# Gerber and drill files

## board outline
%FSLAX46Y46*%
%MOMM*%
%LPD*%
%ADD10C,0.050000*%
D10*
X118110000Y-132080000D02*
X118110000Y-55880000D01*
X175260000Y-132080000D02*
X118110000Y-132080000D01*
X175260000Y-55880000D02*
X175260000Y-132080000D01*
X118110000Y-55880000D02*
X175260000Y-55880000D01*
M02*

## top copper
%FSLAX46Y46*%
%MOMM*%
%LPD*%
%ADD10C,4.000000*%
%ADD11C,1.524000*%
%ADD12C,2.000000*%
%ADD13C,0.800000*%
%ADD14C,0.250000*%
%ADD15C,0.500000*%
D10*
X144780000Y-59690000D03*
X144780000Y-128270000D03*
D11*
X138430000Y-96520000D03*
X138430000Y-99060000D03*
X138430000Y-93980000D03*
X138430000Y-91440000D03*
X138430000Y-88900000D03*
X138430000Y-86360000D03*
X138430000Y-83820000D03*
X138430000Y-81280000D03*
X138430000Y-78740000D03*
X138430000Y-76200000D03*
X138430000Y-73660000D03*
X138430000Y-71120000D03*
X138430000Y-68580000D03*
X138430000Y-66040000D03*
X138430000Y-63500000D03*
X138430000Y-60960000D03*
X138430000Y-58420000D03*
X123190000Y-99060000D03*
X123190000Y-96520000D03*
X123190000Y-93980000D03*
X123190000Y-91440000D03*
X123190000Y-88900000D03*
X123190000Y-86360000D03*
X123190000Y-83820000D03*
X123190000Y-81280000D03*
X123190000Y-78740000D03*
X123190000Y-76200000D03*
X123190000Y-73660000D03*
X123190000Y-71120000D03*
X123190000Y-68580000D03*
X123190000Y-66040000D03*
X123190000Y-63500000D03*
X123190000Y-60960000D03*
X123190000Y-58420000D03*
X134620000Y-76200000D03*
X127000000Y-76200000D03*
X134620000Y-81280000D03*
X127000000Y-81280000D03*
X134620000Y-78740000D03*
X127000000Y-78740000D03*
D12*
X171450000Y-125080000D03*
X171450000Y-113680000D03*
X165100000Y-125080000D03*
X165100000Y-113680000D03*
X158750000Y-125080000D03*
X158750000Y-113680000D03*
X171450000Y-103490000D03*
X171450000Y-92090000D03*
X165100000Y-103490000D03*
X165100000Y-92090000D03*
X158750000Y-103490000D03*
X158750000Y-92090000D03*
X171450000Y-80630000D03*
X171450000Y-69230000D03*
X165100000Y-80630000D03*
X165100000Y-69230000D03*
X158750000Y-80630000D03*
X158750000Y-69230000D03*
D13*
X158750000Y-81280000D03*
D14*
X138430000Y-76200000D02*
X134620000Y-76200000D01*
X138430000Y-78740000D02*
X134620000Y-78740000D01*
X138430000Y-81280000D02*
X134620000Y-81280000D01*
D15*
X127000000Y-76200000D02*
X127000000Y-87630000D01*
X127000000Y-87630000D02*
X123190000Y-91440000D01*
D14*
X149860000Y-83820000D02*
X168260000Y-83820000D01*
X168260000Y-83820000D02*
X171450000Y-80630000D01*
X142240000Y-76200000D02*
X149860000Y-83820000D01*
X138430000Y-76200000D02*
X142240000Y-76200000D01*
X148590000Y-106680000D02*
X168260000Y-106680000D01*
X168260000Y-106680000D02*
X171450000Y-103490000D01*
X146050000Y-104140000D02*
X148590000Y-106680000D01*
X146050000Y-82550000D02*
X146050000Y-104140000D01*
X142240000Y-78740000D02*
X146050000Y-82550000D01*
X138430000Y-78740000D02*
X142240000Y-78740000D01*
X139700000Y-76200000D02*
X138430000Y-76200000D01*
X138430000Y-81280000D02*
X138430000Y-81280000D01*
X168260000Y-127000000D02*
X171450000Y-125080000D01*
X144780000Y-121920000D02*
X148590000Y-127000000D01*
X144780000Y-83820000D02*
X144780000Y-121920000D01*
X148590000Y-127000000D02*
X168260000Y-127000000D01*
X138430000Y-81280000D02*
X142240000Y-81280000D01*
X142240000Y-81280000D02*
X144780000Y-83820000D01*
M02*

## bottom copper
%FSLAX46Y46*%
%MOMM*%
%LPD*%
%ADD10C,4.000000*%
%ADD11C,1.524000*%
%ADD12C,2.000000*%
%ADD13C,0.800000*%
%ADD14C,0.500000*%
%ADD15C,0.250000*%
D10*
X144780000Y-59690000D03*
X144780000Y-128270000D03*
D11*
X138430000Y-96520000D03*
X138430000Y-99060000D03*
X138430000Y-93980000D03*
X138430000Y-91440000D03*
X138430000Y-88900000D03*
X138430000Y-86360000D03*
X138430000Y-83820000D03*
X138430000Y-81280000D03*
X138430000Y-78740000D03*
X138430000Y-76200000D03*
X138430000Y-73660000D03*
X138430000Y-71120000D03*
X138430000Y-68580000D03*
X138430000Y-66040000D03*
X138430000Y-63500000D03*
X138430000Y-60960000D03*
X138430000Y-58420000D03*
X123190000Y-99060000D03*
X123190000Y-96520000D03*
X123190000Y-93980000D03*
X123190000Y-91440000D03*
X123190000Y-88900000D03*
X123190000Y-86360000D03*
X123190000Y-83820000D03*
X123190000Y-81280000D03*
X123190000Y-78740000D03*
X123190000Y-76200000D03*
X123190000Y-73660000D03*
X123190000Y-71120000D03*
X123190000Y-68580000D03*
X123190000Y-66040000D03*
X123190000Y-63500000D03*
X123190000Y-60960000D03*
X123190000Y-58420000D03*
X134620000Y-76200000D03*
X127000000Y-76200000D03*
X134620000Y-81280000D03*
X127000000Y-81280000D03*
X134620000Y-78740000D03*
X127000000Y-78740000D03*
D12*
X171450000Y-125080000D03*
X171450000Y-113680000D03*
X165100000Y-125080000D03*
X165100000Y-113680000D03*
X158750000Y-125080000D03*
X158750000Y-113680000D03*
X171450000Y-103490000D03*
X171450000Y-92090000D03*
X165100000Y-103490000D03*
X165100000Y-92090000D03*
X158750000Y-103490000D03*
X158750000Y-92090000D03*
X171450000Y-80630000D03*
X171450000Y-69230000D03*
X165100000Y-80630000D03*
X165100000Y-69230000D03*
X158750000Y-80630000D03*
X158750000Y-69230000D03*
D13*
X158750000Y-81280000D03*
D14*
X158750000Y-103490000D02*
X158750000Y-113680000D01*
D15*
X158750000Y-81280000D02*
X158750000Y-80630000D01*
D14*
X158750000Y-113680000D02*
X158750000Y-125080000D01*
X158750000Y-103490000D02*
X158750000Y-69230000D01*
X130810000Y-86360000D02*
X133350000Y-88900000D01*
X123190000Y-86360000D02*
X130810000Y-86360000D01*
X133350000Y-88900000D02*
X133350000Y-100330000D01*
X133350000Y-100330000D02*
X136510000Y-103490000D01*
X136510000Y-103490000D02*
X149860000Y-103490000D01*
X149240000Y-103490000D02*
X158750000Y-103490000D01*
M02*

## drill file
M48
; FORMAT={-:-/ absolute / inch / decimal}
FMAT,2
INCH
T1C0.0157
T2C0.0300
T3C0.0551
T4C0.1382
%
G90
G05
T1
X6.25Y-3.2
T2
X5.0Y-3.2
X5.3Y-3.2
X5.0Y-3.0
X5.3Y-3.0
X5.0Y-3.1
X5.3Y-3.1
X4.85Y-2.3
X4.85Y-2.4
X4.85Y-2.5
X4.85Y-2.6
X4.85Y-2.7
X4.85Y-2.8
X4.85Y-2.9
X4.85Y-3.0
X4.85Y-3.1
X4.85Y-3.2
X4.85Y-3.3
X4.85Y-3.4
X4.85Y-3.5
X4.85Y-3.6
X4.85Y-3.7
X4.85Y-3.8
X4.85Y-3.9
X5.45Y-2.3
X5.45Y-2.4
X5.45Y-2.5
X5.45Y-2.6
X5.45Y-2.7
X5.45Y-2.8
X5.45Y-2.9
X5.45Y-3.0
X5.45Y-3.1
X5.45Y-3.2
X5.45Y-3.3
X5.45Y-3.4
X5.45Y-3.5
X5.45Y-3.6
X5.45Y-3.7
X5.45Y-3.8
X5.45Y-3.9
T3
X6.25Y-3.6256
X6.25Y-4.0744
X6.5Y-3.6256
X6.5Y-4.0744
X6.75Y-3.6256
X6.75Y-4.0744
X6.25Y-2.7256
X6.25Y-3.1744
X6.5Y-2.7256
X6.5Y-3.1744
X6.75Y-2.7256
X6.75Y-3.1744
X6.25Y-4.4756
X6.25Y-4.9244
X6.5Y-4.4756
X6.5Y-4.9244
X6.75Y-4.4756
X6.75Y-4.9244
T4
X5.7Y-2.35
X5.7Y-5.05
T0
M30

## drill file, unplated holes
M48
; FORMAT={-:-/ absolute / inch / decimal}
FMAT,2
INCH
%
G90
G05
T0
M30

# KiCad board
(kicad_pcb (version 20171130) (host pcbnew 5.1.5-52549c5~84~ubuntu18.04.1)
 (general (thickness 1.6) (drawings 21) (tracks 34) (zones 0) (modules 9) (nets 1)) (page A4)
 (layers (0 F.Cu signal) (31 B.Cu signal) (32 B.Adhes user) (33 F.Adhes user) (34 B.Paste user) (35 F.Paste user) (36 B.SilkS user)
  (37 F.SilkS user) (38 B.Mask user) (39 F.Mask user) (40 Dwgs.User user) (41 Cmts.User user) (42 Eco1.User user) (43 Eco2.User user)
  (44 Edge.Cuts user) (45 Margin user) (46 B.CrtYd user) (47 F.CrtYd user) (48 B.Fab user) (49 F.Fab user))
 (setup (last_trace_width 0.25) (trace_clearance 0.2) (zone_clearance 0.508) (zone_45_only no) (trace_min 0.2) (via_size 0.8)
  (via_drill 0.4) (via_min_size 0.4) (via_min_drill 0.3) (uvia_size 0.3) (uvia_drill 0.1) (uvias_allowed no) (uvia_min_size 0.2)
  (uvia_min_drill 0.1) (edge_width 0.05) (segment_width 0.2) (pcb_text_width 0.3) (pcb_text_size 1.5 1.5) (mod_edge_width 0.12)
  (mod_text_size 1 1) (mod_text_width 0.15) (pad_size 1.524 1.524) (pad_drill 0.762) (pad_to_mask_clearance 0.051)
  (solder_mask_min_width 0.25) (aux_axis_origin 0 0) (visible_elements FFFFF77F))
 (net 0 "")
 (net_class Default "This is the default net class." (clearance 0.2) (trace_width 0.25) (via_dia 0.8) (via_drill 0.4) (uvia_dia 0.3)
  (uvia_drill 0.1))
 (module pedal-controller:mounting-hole (layer F.Cu) (at 144.78 59.69)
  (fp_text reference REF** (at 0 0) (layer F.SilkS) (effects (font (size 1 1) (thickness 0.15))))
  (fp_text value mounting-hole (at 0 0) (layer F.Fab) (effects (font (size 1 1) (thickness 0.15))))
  (pad 1 thru_hole circle (at 0 0) (size 4 4) (drill 3.51) (layers *.Cu *.Mask)))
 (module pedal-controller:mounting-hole (layer F.Cu) (at 144.78 128.27)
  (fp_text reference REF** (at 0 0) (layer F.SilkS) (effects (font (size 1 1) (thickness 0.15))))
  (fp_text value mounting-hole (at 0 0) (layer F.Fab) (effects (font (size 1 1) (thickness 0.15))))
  (pad 1 thru_hole circle (at 0 0) (size 4 4) (drill 3.51) (layers *.Cu *.Mask)))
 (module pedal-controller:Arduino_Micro (layer F.Cu) (at 123.19 58.42 270)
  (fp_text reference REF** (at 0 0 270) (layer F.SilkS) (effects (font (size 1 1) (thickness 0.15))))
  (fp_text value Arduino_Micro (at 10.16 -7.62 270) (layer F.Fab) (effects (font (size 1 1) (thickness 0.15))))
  (pad 34 thru_hole circle (at 38.1 -15.24 270) (size 1.524 1.524) (drill 0.762) (layers *.Cu *.Mask))
  (pad 33 thru_hole circle (at 40.64 -15.24 270) (size 1.524 1.524) (drill 0.762) (layers *.Cu *.Mask))
  (pad 32 thru_hole circle (at 35.56 -15.24 270) (size 1.524 1.524) (drill 0.762) (layers *.Cu *.Mask))
  (pad 31 thru_hole circle (at 33.02 -15.24 270) (size 1.524 1.524) (drill 0.762) (layers *.Cu *.Mask))
  (pad 30 thru_hole circle (at 30.48 -15.24 270) (size 1.524 1.524) (drill 0.762) (layers *.Cu *.Mask))
  (pad 29 thru_hole circle (at 27.94 -15.24 270) (size 1.524 1.524) (drill 0.762) (layers *.Cu *.Mask))
  (pad 28 thru_hole circle (at 25.4 -15.24 270) (size 1.524 1.524) (drill 0.762) (layers *.Cu *.Mask))
  (pad 27 thru_hole circle (at 22.86 -15.24 270) (size 1.524 1.524) (drill 0.762) (layers *.Cu *.Mask))
  (pad 26 thru_hole circle (at 20.32 -15.24 270) (size 1.524 1.524) (drill 0.762) (layers *.Cu *.Mask))
  (pad 25 thru_hole circle (at 17.78 -15.24 270) (size 1.524 1.524) (drill 0.762) (layers *.Cu *.Mask))
  (pad 24 thru_hole circle (at 15.24 -15.24 270) (size 1.524 1.524) (drill 0.762) (layers *.Cu *.Mask))
  (pad 23 thru_hole circle (at 12.7 -15.24 270) (size 1.524 1.524) (drill 0.762) (layers *.Cu *.Mask))
  (pad 22 thru_hole circle (at 10.16 -15.24 270) (size 1.524 1.524) (drill 0.762) (layers *.Cu *.Mask))
  (pad 21 thru_hole circle (at 7.62 -15.24 270) (size 1.524 1.524) (drill 0.762) (layers *.Cu *.Mask))
  (pad 20 thru_hole circle (at 5.08 -15.24 270) (size 1.524 1.524) (drill 0.762) (layers *.Cu *.Mask))
  (pad 19 thru_hole circle (at 2.54 -15.24 270) (size 1.524 1.524) (drill 0.762) (layers *.Cu *.Mask))
  (pad 18 thru_hole circle (at 0 -15.24 270) (size 1.524 1.524) (drill 0.762) (layers *.Cu *.Mask))
  (pad 17 thru_hole circle (at 40.64 0 270) (size 1.524 1.524) (drill 0.762) (layers *.Cu *.Mask))
  (pad 16 thru_hole circle (at 38.1 0 270) (size 1.524 1.524) (drill 0.762) (layers *.Cu *.Mask))
  (pad 15 thru_hole circle (at 35.56 0 270) (size 1.524 1.524) (drill 0.762) (layers *.Cu *.Mask))
  (pad 14 thru_hole circle (at 33.02 0 270) (size 1.524 1.524) (drill 0.762) (layers *.Cu *.Mask))
  (pad 13 thru_hole circle (at 30.48 0 270) (size 1.524 1.524) (drill 0.762) (layers *.Cu *.Mask))
  (pad 12 thru_hole circle (at 27.94 0 270) (size 1.524 1.524) (drill 0.762) (layers *.Cu *.Mask))
  (pad 11 thru_hole circle (at 25.4 0 270) (size 1.524 1.524) (drill 0.762) (layers *.Cu *.Mask))
  (pad 10 thru_hole circle (at 22.86 0 270) (size 1.524 1.524) (drill 0.762) (layers *.Cu *.Mask))
  (pad 9 thru_hole circle (at 20.32 0 270) (size 1.524 1.524) (drill 0.762) (layers *.Cu *.Mask))
  (pad 8 thru_hole circle (at 17.78 0 270) (size 1.524 1.524) (drill 0.762) (layers *.Cu *.Mask))
  (pad 7 thru_hole circle (at 15.24 0 270) (size 1.524 1.524) (drill 0.762) (layers *.Cu *.Mask))
  (pad 6 thru_hole circle (at 12.7 0 270) (size 1.524 1.524) (drill 0.762) (layers *.Cu *.Mask))
  (pad 5 thru_hole circle (at 10.16 0 270) (size 1.524 1.524) (drill 0.762) (layers *.Cu *.Mask))
  (pad 4 thru_hole circle (at 7.62 0 270) (size 1.524 1.524) (drill 0.762) (layers *.Cu *.Mask))
  (pad 3 thru_hole circle (at 5.08 0 270) (size 1.524 1.524) (drill 0.762) (layers *.Cu *.Mask))
  (pad 2 thru_hole circle (at 2.54 0 270) (size 1.524 1.524) (drill 0.762) (layers *.Cu *.Mask))
  (pad 1 thru_hole circle (at 0 0 270) (size 1.524 1.524) (drill 0.762) (layers *.Cu *.Mask)))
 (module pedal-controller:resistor (layer F.Cu) (at 127 76.2)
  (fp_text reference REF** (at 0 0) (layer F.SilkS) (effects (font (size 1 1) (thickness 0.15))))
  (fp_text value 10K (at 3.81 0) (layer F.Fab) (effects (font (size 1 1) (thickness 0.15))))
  (pad 2 thru_hole circle (at 7.62 0) (size 1.524 1.524) (drill 0.762) (layers *.Cu *.Mask))
  (pad 1 thru_hole circle (at 0 0) (size 1.524 1.524) (drill 0.762) (layers *.Cu *.Mask)))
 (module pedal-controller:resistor (layer F.Cu) (at 127 81.28)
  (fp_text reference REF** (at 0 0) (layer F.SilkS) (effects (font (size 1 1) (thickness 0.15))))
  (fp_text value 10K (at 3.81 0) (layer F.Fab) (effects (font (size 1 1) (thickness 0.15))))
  (pad 2 thru_hole circle (at 7.62 0) (size 1.524 1.524) (drill 0.762) (layers *.Cu *.Mask))
  (pad 1 thru_hole circle (at 0 0) (size 1.524 1.524) (drill 0.762) (layers *.Cu *.Mask)))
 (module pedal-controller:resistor (layer F.Cu) (at 127 78.74)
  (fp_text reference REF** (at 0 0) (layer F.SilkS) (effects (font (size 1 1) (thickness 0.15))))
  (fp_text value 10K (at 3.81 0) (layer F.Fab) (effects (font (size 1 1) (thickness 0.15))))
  (pad 2 thru_hole circle (at 7.62 0) (size 1.524 1.524) (drill 0.762) (layers *.Cu *.Mask))
  (pad 1 thru_hole circle (at 0 0) (size 1.524 1.524) (drill 0.762) (layers *.Cu *.Mask)))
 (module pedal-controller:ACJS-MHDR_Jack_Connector (layer F.Cu) (at 165.1 119.38)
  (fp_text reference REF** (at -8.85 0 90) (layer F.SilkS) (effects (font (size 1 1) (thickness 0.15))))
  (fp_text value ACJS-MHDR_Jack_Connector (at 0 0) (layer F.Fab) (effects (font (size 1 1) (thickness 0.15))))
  (pad 3 thru_hole circle (at 6.35 5.7) (size 2 2) (drill 1.4) (layers *.Cu *.Mask))
  (pad 4 thru_hole circle (at 6.35 -5.7) (size 2 2) (drill 1.4) (layers *.Cu *.Mask))
  (pad 2 thru_hole circle (at 0 5.7) (size 2 2) (drill 1.4) (layers *.Cu *.Mask))
  (pad 5 thru_hole circle (at 0 -5.7) (size 2 2) (drill 1.4) (layers *.Cu *.Mask))
  (pad 1 thru_hole circle (at -6.35 5.7) (size 2 2) (drill 1.4) (layers *.Cu *.Mask))
  (pad 6 thru_hole circle (at -6.35 -5.7) (size 2 2) (drill 1.4) (layers *.Cu *.Mask)))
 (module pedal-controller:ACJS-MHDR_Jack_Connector (layer F.Cu) (at 165.1 97.79)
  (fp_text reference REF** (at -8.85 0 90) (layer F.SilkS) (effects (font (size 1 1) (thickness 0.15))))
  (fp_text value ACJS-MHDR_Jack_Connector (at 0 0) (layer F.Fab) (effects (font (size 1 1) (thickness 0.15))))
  (pad 3 thru_hole circle (at 6.35 5.7) (size 2 2) (drill 1.4) (layers *.Cu *.Mask))
  (pad 4 thru_hole circle (at 6.35 -5.7) (size 2 2) (drill 1.4) (layers *.Cu *.Mask))
  (pad 2 thru_hole circle (at 0 5.7) (size 2 2) (drill 1.4) (layers *.Cu *.Mask))
  (pad 5 thru_hole circle (at 0 -5.7) (size 2 2) (drill 1.4) (layers *.Cu *.Mask))
  (pad 1 thru_hole circle (at -6.35 5.7) (size 2 2) (drill 1.4) (layers *.Cu *.Mask))
  (pad 6 thru_hole circle (at -6.35 -5.7) (size 2 2) (drill 1.4) (layers *.Cu *.Mask)))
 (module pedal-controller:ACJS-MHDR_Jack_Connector (layer F.Cu) (at 165.1 74.93)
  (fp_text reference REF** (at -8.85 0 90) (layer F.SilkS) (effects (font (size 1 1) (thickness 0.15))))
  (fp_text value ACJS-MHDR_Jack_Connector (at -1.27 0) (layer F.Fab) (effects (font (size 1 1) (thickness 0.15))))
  (pad 3 thru_hole circle (at 6.35 5.7) (size 2 2) (drill 1.4) (layers *.Cu *.Mask))
  (pad 4 thru_hole circle (at 6.35 -5.7) (size 2 2) (drill 1.4) (layers *.Cu *.Mask))
  (pad 2 thru_hole circle (at 0 5.7) (size 2 2) (drill 1.4) (layers *.Cu *.Mask))
  (pad 5 thru_hole circle (at 0 -5.7) (size 2 2) (drill 1.4) (layers *.Cu *.Mask))
  (pad 1 thru_hole circle (at -6.35 5.7) (size 2 2) (drill 1.4) (layers *.Cu *.Mask))
  (pad 6 thru_hole circle (at -6.35 -5.7) (size 2 2) (drill 1.4) (layers *.Cu *.Mask)))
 (gr_line (start 118.11 132.08) (end 118.11 55.88) (layer Edge.Cuts) (width 0.05))
 (gr_line (start 175.26 132.08) (end 118.11 132.08) (layer Edge.Cuts) (width 0.05))
 (gr_line (start 175.26 55.88) (end 175.26 132.08) (layer Edge.Cuts) (width 0.05))
 (gr_line (start 118.11 55.88) (end 175.26 55.88) (layer Edge.Cuts) (width 0.05))
 (segment (start 158.75 103.49) (end 158.75 113.68) (width 0.5) (layer B.Cu) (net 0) (status 30))
 (segment (start 138.43 76.2) (end 134.62 76.2) (width 0.25) (layer F.Cu) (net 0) (status 30))
 (segment (start 138.43 78.74) (end 134.62 78.74) (width 0.25) (layer F.Cu) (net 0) (status 30))
 (segment (start 138.43 81.28) (end 134.62 81.28) (width 0.25) (layer F.Cu) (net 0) (status 30))
 (segment (start 158.75 81.28) (end 158.75 80.63) (width 0.25) (layer B.Cu) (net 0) (status 30))
 (segment (start 158.75 113.68) (end 158.75 125.08) (width 0.5) (layer B.Cu) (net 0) (status 30))
 (segment (start 158.75 103.49) (end 158.75 69.23) (width 0.5) (layer B.Cu) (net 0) (status 30))
 (segment (start 130.81 86.36) (end 133.35 88.9) (width 0.5) (layer B.Cu) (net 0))
 (segment (start 123.19 86.36) (end 130.81 86.36) (width 0.5) (layer B.Cu) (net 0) (status 10))
 (segment (start 133.35 88.9) (end 133.35 100.33) (width 0.5) (layer B.Cu) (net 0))
 (segment (start 133.35 100.33) (end 136.51 103.49) (width 0.5) (layer B.Cu) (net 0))
 (segment (start 136.51 103.49) (end 149.86 103.49) (width 0.5) (layer B.Cu) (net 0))
 (segment (start 127 76.2) (end 127 87.63) (width 0.5) (layer F.Cu) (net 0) (status 10))
 (segment (start 127 87.63) (end 123.19 91.44) (width 0.5) (layer F.Cu) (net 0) (status 20))
 (segment (start 149.86 83.82) (end 168.26 83.82) (width 0.25) (layer F.Cu) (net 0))
 (segment (start 168.26 83.82) (end 171.45 80.63) (width 0.25) (layer F.Cu) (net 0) (status 20))
 (segment (start 142.24 76.2) (end 149.86 83.82) (width 0.25) (layer F.Cu) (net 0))
 (segment (start 138.43 76.2) (end 142.24 76.2) (width 0.25) (layer F.Cu) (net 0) (status 10))
 (segment (start 148.59 106.68) (end 168.26 106.68) (width 0.25) (layer F.Cu) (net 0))
 (segment (start 168.26 106.68) (end 171.45 103.49) (width 0.25) (layer F.Cu) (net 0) (status 20))
 (segment (start 146.05 104.14) (end 148.59 106.68) (width 0.25) (layer F.Cu) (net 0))
 (segment (start 146.05 82.55) (end 146.05 104.14) (width 0.25) (layer F.Cu) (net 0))
 (segment (start 142.24 78.74) (end 146.05 82.55) (width 0.25) (layer F.Cu) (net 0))
 (segment (start 138.43 78.74) (end 142.24 78.74) (width 0.25) (layer F.Cu) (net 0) (status 10))
 (segment (start 149.24 103.49) (end 158.75 103.49) (width 0.5) (layer B.Cu) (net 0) (status 20))
 (segment (start 139.7 76.2) (end 138.43 76.2) (width 0.25) (layer F.Cu) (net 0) (status 20))
 (segment (start 138.43 81.28) (end 138.43 81.28) (width 0.25) (layer F.Cu) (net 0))
 (via (at 158.75 81.28) (size 0.8) (drill 0.4) (layers F.Cu B.Cu) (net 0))
 (segment (start 168.26 127) (end 171.45 125.08) (width 0.25) (layer F.Cu) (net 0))
 (segment (start 144.78 121.92) (end 148.59 127) (width 0.25) (layer F.Cu) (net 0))
 (segment (start 144.78 83.82) (end 144.78 121.92) (width 0.25) (layer F.Cu) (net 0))
 (segment (start 148.59 127) (end 168.26 127) (width 0.25) (layer F.Cu) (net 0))
 (segment (start 138.43 81.28) (end 142.24 81.28) (width 0.25) (layer F.Cu) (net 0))
 (segment (start 142.24 81.28) (end 144.78 83.82) (width 0.25) (layer F.Cu) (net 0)))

